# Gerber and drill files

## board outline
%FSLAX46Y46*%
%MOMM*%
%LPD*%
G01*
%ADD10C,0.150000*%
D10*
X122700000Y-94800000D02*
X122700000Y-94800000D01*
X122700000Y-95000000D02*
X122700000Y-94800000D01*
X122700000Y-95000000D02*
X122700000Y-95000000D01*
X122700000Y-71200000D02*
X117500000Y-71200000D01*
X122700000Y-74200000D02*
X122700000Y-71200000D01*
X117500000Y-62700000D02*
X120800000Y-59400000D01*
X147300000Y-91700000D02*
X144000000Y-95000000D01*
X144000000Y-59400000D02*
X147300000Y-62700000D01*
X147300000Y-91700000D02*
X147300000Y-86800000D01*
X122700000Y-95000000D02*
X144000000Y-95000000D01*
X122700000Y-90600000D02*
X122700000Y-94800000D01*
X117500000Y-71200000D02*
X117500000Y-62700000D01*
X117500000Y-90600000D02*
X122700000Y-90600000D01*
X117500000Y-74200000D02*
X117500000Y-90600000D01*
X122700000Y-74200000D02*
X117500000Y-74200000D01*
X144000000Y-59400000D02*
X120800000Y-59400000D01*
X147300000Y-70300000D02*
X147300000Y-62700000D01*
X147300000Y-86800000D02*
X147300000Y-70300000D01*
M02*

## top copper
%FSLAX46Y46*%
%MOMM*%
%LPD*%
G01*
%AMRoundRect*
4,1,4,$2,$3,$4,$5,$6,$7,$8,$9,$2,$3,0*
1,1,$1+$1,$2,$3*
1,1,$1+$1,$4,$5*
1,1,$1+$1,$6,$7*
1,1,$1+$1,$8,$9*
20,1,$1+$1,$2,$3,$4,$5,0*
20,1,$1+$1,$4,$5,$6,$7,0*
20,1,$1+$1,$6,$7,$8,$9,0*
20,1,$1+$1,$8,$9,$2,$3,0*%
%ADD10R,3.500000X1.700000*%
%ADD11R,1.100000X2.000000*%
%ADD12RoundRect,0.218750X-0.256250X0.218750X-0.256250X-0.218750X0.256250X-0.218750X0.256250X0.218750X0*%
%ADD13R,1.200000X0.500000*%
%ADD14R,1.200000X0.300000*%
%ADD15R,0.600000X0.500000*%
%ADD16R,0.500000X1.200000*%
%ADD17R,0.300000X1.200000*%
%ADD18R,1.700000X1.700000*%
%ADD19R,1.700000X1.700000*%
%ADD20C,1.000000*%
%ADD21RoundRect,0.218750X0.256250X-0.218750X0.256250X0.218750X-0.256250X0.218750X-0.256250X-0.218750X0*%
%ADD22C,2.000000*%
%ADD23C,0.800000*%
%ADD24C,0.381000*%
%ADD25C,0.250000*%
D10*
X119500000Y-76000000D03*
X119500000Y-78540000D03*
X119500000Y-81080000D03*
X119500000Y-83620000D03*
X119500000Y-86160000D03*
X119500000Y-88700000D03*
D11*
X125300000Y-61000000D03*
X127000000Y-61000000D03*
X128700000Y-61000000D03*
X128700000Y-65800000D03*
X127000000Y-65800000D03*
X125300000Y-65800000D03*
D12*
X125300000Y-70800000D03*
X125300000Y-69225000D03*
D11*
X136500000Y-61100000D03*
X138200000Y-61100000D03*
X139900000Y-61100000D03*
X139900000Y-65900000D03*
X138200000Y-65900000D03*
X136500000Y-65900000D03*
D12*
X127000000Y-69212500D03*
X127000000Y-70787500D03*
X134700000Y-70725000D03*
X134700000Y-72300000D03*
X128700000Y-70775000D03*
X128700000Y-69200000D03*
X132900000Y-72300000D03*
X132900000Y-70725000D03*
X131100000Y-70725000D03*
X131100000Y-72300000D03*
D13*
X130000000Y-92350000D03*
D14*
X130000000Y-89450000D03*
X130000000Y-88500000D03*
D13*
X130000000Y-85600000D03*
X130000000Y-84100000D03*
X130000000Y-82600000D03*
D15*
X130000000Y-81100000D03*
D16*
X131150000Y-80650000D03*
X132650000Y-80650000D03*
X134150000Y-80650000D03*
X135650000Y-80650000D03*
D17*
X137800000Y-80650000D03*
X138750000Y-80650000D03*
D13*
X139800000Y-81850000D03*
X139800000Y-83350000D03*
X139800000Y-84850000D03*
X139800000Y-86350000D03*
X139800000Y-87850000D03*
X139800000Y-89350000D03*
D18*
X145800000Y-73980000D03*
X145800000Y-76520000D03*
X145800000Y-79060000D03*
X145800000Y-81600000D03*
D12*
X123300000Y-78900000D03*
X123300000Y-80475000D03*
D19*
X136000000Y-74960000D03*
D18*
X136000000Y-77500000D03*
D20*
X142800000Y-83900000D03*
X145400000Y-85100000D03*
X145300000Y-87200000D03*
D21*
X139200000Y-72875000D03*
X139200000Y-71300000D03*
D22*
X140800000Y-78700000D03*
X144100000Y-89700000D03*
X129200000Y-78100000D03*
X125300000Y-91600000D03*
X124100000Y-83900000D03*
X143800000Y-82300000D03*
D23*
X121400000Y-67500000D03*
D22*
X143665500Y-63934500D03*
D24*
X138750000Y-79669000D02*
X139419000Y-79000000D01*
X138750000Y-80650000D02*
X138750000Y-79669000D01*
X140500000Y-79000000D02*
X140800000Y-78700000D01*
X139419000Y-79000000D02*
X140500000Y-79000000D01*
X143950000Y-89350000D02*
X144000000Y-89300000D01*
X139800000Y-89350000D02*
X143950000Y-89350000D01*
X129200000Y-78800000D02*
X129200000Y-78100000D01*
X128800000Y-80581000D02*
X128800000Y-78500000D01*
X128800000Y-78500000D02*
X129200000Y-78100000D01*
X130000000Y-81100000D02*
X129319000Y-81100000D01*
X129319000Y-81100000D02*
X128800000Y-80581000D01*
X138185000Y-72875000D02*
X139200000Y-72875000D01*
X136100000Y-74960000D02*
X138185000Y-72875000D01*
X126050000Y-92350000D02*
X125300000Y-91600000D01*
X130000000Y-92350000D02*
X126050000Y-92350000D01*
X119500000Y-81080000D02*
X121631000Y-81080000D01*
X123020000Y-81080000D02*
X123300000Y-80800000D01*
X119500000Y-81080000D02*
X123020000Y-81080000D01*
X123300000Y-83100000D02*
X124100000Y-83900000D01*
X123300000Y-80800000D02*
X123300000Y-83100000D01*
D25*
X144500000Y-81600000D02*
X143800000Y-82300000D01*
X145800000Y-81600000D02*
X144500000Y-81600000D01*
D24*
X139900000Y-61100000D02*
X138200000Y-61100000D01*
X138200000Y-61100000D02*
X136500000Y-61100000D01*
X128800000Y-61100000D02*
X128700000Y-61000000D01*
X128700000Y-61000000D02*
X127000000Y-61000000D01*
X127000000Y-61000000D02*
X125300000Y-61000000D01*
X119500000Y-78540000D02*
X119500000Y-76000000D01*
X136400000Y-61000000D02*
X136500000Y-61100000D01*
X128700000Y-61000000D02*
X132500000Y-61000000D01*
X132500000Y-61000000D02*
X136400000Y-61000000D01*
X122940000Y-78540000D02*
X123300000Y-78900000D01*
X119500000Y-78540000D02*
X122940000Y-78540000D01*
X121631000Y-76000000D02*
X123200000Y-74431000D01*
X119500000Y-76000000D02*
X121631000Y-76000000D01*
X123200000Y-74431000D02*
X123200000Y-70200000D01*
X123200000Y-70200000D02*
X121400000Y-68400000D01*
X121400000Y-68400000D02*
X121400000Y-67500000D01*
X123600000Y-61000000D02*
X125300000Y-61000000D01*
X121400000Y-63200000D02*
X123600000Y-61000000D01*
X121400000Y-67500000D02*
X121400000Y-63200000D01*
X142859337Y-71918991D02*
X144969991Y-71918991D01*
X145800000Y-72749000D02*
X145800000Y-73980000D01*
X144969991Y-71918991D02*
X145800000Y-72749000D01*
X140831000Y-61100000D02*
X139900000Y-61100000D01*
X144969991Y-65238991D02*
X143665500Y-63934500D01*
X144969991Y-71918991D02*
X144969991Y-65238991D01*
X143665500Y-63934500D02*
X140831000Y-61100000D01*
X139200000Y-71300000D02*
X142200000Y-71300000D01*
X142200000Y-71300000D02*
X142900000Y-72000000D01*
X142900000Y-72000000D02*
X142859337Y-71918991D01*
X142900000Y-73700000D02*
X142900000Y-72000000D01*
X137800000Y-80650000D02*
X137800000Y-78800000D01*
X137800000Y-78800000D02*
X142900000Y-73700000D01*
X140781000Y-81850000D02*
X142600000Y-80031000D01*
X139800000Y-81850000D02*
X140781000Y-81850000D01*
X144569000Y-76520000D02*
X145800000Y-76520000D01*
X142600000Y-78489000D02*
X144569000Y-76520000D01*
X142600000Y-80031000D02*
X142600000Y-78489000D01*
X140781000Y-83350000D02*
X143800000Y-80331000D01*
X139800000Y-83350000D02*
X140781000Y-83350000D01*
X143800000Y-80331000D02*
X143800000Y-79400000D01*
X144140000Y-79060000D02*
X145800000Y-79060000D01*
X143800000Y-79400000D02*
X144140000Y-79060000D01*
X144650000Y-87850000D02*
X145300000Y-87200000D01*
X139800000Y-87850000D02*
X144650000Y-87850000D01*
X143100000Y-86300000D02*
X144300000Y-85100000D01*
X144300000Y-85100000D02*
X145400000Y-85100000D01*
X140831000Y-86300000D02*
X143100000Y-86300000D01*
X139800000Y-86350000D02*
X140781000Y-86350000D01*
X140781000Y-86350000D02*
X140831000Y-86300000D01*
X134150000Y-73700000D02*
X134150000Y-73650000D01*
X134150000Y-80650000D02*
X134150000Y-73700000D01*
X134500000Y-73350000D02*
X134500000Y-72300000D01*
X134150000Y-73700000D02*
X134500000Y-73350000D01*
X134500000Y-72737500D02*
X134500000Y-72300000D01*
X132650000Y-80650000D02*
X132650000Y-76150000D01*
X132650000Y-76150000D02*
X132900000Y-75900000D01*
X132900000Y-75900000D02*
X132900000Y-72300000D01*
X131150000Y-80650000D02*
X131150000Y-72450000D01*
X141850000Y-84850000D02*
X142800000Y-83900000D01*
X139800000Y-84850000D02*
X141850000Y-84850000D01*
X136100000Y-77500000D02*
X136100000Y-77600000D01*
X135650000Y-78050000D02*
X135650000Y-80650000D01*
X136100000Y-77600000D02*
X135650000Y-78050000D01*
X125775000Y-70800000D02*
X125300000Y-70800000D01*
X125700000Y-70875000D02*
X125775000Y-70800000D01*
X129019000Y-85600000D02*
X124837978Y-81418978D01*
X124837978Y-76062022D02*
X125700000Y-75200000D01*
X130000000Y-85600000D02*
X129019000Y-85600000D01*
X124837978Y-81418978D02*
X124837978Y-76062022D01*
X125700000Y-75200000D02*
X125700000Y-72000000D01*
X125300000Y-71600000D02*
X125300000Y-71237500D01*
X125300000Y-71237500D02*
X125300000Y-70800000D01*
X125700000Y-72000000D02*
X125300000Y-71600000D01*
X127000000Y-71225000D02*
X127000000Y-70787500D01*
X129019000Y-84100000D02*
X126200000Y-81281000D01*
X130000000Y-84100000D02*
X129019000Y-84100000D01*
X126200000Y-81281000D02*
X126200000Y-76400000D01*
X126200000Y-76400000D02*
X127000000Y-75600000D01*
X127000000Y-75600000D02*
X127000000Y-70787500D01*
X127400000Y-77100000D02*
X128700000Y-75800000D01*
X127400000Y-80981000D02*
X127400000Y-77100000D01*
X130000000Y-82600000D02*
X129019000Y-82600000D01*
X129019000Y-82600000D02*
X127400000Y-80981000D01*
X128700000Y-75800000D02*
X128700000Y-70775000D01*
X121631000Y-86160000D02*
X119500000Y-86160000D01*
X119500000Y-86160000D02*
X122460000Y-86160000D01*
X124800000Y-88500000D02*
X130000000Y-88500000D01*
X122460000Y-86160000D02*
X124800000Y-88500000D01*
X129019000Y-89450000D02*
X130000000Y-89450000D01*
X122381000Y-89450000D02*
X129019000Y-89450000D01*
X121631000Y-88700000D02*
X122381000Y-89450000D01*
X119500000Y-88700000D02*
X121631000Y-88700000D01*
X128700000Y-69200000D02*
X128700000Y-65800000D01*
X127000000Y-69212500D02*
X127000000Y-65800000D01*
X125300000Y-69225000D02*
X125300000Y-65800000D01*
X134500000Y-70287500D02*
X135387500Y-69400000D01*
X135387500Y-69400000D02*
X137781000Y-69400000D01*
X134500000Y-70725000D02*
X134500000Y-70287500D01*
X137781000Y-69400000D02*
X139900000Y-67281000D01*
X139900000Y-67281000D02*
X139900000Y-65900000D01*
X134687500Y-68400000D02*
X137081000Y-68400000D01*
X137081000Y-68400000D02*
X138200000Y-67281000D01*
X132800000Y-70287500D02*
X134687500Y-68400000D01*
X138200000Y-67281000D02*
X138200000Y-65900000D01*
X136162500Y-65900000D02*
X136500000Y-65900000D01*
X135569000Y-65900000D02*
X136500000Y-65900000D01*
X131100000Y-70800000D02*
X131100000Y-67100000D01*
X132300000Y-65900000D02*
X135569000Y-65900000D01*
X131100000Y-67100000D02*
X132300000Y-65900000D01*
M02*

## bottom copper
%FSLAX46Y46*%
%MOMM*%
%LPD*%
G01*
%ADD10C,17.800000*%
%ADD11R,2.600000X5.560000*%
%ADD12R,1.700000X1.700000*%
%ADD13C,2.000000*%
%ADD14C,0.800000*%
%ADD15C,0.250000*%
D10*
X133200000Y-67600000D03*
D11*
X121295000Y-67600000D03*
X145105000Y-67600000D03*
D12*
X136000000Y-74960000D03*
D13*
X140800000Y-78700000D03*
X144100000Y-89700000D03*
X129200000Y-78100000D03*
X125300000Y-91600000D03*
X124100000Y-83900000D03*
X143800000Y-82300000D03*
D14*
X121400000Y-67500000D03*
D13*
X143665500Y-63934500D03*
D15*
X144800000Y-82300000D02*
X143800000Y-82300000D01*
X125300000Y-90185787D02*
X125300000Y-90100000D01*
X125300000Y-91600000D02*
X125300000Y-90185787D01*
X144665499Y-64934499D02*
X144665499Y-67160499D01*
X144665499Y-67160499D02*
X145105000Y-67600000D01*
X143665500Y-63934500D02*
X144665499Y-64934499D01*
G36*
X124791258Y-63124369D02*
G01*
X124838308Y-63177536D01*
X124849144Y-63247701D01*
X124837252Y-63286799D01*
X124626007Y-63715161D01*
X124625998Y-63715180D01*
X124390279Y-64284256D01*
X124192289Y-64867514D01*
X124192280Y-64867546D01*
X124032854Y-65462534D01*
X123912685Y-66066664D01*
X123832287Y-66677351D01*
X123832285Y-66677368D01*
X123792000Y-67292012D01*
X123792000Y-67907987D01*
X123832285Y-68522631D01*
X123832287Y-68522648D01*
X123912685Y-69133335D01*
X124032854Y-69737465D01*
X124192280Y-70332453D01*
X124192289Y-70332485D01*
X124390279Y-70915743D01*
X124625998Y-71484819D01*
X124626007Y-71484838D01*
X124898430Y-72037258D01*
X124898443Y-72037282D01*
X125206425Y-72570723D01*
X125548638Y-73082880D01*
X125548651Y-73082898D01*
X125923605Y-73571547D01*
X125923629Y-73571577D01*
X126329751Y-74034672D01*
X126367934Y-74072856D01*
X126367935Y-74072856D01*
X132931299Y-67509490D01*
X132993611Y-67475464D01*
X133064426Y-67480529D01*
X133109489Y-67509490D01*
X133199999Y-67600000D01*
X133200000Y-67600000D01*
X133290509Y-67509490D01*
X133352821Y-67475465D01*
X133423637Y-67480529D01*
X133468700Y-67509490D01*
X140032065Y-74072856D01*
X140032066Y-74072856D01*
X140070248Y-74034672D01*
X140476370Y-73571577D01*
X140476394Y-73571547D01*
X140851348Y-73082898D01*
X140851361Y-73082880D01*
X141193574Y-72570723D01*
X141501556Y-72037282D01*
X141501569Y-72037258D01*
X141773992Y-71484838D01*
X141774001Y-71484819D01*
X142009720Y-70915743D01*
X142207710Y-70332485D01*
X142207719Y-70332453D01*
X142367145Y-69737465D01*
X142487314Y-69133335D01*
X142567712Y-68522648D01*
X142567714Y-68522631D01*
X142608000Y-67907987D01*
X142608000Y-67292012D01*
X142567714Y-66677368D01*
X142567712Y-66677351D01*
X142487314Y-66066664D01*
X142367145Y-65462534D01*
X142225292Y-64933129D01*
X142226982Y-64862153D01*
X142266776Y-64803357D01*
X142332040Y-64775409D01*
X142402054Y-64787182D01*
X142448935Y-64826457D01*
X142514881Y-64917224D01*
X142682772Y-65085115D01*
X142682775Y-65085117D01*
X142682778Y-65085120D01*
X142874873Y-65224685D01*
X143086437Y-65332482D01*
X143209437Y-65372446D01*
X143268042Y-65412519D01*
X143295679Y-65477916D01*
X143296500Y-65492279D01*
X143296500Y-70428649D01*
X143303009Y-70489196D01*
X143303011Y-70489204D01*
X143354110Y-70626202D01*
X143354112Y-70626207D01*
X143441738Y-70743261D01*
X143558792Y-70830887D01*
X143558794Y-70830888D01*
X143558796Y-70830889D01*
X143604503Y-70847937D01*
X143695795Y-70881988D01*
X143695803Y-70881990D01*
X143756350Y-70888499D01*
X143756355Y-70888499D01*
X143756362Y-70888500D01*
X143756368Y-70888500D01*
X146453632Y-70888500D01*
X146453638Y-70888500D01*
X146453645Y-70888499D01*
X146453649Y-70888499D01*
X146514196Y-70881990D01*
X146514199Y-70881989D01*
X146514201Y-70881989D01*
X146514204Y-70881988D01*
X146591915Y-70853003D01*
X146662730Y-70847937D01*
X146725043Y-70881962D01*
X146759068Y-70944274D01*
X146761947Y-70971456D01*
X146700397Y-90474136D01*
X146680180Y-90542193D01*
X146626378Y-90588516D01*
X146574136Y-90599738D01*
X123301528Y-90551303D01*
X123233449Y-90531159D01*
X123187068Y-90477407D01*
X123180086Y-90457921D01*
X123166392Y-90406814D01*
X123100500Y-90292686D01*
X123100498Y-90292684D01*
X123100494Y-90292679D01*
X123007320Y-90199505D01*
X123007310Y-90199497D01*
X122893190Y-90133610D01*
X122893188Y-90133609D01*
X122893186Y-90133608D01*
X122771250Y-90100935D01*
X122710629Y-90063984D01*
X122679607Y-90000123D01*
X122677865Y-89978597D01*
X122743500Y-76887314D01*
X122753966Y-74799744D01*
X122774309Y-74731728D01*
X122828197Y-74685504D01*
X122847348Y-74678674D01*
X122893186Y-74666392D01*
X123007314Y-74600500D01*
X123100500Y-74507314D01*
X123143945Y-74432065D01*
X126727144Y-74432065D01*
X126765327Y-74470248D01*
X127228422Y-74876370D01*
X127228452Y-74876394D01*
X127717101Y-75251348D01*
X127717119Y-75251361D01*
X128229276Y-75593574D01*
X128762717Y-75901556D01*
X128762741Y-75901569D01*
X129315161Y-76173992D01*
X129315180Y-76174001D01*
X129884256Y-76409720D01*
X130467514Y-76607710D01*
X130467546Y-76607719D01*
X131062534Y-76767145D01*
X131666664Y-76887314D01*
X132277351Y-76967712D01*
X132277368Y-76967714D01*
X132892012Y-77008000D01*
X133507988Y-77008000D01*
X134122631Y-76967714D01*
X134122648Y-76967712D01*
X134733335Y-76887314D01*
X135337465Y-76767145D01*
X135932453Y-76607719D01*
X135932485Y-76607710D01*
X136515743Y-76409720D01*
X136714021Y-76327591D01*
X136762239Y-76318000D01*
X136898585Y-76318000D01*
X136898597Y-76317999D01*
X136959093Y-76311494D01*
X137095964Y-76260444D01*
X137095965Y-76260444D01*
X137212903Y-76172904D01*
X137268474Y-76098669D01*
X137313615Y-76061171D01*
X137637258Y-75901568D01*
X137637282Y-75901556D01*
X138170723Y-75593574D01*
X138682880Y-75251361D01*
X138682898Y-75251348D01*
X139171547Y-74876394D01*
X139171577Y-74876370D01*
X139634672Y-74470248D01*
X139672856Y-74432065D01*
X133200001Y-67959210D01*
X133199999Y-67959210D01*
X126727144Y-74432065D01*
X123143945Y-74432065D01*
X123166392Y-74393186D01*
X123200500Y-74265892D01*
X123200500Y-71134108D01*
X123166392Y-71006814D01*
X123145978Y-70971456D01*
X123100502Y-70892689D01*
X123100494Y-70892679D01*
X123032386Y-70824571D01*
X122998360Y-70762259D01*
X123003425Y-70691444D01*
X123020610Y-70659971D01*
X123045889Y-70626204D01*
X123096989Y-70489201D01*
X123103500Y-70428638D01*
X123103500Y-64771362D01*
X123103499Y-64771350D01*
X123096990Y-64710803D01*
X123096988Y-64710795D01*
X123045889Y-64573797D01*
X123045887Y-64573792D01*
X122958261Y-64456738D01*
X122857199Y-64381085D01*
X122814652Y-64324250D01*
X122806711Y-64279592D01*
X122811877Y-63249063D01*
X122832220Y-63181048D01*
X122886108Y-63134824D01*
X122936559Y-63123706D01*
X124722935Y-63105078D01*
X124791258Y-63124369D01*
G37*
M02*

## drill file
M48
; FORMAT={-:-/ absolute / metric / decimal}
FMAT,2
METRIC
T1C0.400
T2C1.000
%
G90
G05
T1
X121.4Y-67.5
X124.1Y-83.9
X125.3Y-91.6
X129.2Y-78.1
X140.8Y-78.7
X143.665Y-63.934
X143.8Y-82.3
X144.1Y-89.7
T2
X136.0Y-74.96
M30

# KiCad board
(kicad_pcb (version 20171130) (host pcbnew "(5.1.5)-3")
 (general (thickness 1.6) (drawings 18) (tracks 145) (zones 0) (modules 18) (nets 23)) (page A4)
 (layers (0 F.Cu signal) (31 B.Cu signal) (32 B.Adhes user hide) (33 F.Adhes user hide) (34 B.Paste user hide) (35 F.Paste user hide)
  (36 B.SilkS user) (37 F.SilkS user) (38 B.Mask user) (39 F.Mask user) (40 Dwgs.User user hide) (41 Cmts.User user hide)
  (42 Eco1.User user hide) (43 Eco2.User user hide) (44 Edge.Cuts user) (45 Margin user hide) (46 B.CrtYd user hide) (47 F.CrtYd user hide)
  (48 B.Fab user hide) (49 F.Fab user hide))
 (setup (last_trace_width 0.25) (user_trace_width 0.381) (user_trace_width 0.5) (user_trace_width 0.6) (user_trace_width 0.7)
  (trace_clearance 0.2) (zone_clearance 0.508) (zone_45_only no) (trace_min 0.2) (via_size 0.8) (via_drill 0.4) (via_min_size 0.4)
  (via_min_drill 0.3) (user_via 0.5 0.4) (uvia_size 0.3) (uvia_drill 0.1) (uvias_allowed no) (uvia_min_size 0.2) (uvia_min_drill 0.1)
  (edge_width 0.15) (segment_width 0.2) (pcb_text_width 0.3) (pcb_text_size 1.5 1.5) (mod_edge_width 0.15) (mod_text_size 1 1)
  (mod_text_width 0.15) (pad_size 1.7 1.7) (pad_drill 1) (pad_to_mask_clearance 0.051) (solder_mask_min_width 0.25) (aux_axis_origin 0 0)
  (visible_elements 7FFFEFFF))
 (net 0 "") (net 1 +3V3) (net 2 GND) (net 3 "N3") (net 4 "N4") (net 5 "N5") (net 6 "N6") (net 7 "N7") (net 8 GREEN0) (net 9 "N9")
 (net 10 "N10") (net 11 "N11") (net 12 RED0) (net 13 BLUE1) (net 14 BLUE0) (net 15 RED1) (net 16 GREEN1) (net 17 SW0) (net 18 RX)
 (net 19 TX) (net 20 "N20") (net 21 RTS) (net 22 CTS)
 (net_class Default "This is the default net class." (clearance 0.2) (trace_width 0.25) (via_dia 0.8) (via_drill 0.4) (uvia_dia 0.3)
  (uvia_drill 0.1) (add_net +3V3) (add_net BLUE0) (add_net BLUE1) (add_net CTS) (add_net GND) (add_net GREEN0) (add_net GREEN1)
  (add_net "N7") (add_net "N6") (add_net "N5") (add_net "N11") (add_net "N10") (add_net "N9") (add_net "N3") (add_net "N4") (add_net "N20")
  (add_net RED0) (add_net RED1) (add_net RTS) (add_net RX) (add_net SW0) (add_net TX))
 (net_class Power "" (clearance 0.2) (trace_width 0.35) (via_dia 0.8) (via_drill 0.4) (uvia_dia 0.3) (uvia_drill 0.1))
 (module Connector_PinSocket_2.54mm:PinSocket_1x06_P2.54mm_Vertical (layer F.Cu) (at 119.5 76)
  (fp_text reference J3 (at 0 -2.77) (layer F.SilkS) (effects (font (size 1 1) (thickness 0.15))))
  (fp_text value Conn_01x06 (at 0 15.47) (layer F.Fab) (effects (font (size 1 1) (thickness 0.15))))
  (pad 1 smd rect (at 0 0) (size 3.5 1.7) (layers F.Cu F.Paste F.Mask) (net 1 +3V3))
  (pad 2 smd rect (at 0 2.54) (size 3.5 1.7) (layers F.Cu F.Paste F.Mask) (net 1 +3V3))
  (pad 3 smd rect (at 0 5.08) (size 3.5 1.7) (layers F.Cu F.Paste F.Mask) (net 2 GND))
  (pad 4 smd rect (at 0 7.62) (size 3.5 1.7) (layers F.Cu F.Paste F.Mask))
  (pad 5 smd rect (at 0 10.16) (size 3.5 1.7) (layers F.Cu F.Paste F.Mask) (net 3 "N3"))
  (pad 6 smd rect (at 0 12.7) (size 3.5 1.7) (layers F.Cu F.Paste F.Mask) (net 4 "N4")))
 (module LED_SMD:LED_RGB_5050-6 (layer F.Cu) (at 127 63.4 90)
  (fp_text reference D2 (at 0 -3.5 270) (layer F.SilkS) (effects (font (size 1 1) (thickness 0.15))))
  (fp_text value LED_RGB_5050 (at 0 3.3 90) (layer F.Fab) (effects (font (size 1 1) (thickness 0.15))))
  (pad 6 smd rect (at 2.4 -1.7 180) (size 1.1 2) (layers F.Cu F.Paste F.Mask) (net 1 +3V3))
  (pad 5 smd rect (at 2.4 0 180) (size 1.1 2) (layers F.Cu F.Paste F.Mask) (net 1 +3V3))
  (pad 4 smd rect (at 2.4 1.7 180) (size 1.1 2) (layers F.Cu F.Paste F.Mask) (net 1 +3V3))
  (pad 3 smd rect (at -2.4 1.7 180) (size 1.1 2) (layers F.Cu F.Paste F.Mask) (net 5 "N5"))
  (pad 2 smd rect (at -2.4 0 180) (size 1.1 2) (layers F.Cu F.Paste F.Mask) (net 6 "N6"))
  (pad 1 smd rect (at -2.4 -1.7 180) (size 1.1 2) (layers F.Cu F.Paste F.Mask) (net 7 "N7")))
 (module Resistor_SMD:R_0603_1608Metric (layer F.Cu) (at 125.3 70.0125 270)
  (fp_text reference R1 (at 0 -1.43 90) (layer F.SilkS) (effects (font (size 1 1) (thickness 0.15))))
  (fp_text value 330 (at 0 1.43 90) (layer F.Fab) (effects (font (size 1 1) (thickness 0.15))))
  (pad 2 smd roundrect (at 0.7875 0 270) (size 0.875 0.95) (layers F.Cu F.Paste F.Mask) (roundrect_rratio 0.25) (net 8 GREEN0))
  (pad 1 smd roundrect (at -0.7875 0 270) (size 0.875 0.95) (layers F.Cu F.Paste F.Mask) (roundrect_rratio 0.25) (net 7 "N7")))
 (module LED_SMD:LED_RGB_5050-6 (layer F.Cu) (at 138.2 63.5 90)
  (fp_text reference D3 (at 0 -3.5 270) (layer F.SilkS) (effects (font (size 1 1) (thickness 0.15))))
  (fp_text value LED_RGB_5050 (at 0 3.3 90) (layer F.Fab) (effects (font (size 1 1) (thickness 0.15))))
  (pad 6 smd rect (at 2.4 -1.7 180) (size 1.1 2) (layers F.Cu F.Paste F.Mask) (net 1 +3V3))
  (pad 5 smd rect (at 2.4 0 180) (size 1.1 2) (layers F.Cu F.Paste F.Mask) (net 1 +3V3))
  (pad 4 smd rect (at 2.4 1.7 180) (size 1.1 2) (layers F.Cu F.Paste F.Mask) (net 1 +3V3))
  (pad 3 smd rect (at -2.4 1.7 180) (size 1.1 2) (layers F.Cu F.Paste F.Mask) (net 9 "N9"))
  (pad 2 smd rect (at -2.4 0 180) (size 1.1 2) (layers F.Cu F.Paste F.Mask) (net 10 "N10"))
  (pad 1 smd rect (at -2.4 -1.7 180) (size 1.1 2) (layers F.Cu F.Paste F.Mask) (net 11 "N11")))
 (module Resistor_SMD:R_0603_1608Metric (layer F.Cu) (at 127 70 270)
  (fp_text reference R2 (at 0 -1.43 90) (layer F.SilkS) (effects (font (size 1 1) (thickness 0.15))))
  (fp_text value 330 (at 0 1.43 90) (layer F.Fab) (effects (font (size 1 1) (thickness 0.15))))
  (pad 1 smd roundrect (at -0.7875 0 270) (size 0.875 0.95) (layers F.Cu F.Paste F.Mask) (roundrect_rratio 0.25) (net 6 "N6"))
  (pad 2 smd roundrect (at 0.7875 0 270) (size 0.875 0.95) (layers F.Cu F.Paste F.Mask) (roundrect_rratio 0.25) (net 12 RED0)))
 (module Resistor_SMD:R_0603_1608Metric (layer F.Cu) (at 134.7 71.5125 270)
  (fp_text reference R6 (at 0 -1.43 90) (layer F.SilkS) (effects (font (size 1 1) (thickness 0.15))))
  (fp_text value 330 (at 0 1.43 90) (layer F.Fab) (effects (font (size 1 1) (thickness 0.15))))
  (pad 1 smd roundrect (at -0.7875 0 270) (size 0.875 0.95) (layers F.Cu F.Paste F.Mask) (roundrect_rratio 0.25) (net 9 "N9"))
  (pad 2 smd roundrect (at 0.7875 0 270) (size 0.875 0.95) (layers F.Cu F.Paste F.Mask) (roundrect_rratio 0.25) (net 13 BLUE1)))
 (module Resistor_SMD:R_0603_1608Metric (layer F.Cu) (at 128.7 69.9875 270)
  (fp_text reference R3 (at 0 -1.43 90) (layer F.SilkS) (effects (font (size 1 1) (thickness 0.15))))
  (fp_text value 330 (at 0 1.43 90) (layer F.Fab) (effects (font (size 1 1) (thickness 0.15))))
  (pad 2 smd roundrect (at 0.7875 0 270) (size 0.875 0.95) (layers F.Cu F.Paste F.Mask) (roundrect_rratio 0.25) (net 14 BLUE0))
  (pad 1 smd roundrect (at -0.7875 0 270) (size 0.875 0.95) (layers F.Cu F.Paste F.Mask) (roundrect_rratio 0.25) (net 5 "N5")))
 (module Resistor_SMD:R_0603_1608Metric (layer F.Cu) (at 132.9 71.5125 270)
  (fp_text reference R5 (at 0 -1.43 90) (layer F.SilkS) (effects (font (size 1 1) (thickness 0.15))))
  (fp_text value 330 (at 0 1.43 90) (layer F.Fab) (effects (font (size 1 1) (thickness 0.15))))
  (pad 2 smd roundrect (at 0.7875 0 270) (size 0.875 0.95) (layers F.Cu F.Paste F.Mask) (roundrect_rratio 0.25) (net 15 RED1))
  (pad 1 smd roundrect (at -0.7875 0 270) (size 0.875 0.95) (layers F.Cu F.Paste F.Mask) (roundrect_rratio 0.25) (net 10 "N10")))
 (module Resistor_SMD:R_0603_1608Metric (layer F.Cu) (at 131.1 71.5125 270)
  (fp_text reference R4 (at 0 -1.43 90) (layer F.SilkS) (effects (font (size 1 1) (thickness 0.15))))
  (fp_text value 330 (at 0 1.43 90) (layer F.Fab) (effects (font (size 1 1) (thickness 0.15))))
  (pad 1 smd roundrect (at -0.7875 0 270) (size 0.875 0.95) (layers F.Cu F.Paste F.Mask) (roundrect_rratio 0.25) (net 11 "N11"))
  (pad 2 smd roundrect (at 0.7875 0 270) (size 0.875 0.95) (layers F.Cu F.Paste F.Mask) (roundrect_rratio 0.25) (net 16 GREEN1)))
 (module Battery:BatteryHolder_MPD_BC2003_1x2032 (layer B.Cu) (at 133.2 67.6 180)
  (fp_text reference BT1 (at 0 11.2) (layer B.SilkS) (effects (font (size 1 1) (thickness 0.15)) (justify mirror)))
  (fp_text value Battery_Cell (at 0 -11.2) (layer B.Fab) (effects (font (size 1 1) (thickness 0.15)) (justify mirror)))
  (pad 2 smd circle (at 0 0 180) (size 17.8 17.8) (layers B.Cu B.Mask) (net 2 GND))
  (pad 1 smd rect (at 11.905 0 180) (size 2.6 5.56) (layers B.Cu B.Paste B.Mask) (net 1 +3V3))
  (pad 1 smd rect (at -11.905 0 180) (size 2.6 5.56) (layers B.Cu B.Paste B.Mask) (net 1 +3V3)))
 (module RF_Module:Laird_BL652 (layer F.Cu) (at 134.9 86.5 90)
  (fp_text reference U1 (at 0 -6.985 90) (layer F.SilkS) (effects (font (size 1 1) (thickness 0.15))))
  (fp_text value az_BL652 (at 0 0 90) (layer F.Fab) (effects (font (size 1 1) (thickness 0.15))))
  (pad 1 smd rect (at -5.85 -4.9 180) (size 1.2 0.5) (layers F.Cu F.Paste F.Mask) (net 2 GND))
  (pad 5 smd rect (at -2.95 -4.9 180) (size 1.2 0.3) (layers F.Cu F.Paste F.Mask) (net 4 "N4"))
  (pad 6 smd rect (at -2 -4.9 180) (size 1.2 0.3) (layers F.Cu F.Paste F.Mask) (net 3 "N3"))
  (pad 10 smd rect (at 0.9 -4.9 180) (size 1.2 0.5) (layers F.Cu F.Paste F.Mask) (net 8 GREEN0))
  (pad 12 smd rect (at 2.4 -4.9 180) (size 1.2 0.5) (layers F.Cu F.Paste F.Mask) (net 12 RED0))
  (pad 14 smd rect (at 3.9 -4.9 180) (size 1.2 0.5) (layers F.Cu F.Paste F.Mask) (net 14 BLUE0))
  (pad 16 smd rect (at 5.4 -4.9 180) (size 0.6 0.5) (layers F.Cu F.Paste F.Mask) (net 2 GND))
  (pad 17 smd rect (at 5.85 -3.75 90) (size 1.2 0.5) (layers F.Cu F.Paste F.Mask) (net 16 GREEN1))
  (pad 19 smd rect (at 5.85 -2.25 90) (size 1.2 0.5) (layers F.Cu F.Paste F.Mask) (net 15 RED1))
  (pad 21 smd rect (at 5.85 -0.75 90) (size 1.2 0.5) (layers F.Cu F.Paste F.Mask) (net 13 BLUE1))
  (pad 23 smd rect (at 5.85 0.75 90) (size 1.2 0.5) (layers F.Cu F.Paste F.Mask) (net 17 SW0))
  (pad 26 smd rect (at 5.85 2.9 90) (size 1.2 0.3) (layers F.Cu F.Paste F.Mask) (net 1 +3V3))
  (pad 27 smd rect (at 5.85 3.85 90) (size 1.2 0.3) (layers F.Cu F.Paste F.Mask) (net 2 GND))
  (pad 29 smd rect (at 4.65 4.9 180) (size 1.2 0.5) (layers F.Cu F.Paste F.Mask) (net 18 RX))
  (pad 31 smd rect (at 3.15 4.9 180) (size 1.2 0.5) (layers F.Cu F.Paste F.Mask) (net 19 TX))
  (pad 33 smd rect (at 1.65 4.9 180) (size 1.2 0.5) (layers F.Cu F.Paste F.Mask) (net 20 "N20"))
  (pad 35 smd rect (at 0.15 4.9 180) (size 1.2 0.5) (layers F.Cu F.Paste F.Mask) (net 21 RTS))
  (pad 37 smd rect (at -1.35 4.9 180) (size 1.2 0.5) (layers F.Cu F.Paste F.Mask) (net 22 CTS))
  (pad 39 smd rect (at -2.85 4.9 180) (size 1.2 0.5) (layers F.Cu F.Paste F.Mask) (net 2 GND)))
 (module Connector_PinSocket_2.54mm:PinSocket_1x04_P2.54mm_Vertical (layer F.Cu) (at 145.8 73.98)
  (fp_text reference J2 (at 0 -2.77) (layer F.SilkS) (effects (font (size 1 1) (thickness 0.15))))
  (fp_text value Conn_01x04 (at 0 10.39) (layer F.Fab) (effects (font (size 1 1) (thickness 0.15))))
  (pad 1 smd rect (at 0 0) (size 1.7 1.7) (layers F.Cu F.Paste F.Mask) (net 1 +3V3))
  (pad 2 smd rect (at 0 2.54) (size 1.7 1.7) (layers F.Cu F.Paste F.Mask) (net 18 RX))
  (pad 3 smd rect (at 0 5.08) (size 1.7 1.7) (layers F.Cu F.Paste F.Mask) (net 19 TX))
  (pad 4 smd rect (at 0 7.62) (size 1.7 1.7) (layers F.Cu F.Paste F.Mask) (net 2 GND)))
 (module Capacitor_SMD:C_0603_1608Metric (layer F.Cu) (at 123.3 79.6875 270)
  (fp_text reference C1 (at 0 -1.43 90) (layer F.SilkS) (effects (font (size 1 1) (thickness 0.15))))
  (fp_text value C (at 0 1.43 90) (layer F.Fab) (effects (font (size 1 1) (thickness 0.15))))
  (pad 1 smd roundrect (at -0.7875 0 270) (size 0.875 0.95) (layers F.Cu F.Paste F.Mask) (roundrect_rratio 0.25) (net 1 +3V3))
  (pad 2 smd roundrect (at 0.7875 0 270) (size 0.875 0.95) (layers F.Cu F.Paste F.Mask) (roundrect_rratio 0.25) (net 2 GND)))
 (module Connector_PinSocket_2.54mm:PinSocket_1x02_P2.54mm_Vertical (layer F.Cu) (at 136 77.5 180)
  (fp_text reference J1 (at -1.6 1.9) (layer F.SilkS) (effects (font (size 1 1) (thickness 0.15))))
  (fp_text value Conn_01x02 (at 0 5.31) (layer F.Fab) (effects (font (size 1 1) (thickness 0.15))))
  (pad 2 thru_hole rect (at 0 2.54 180) (size 1.7 1.7) (drill 1) (layers *.Cu *.Mask) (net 2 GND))
  (pad 1 smd rect (at 0 0 180) (size 1.7 1.7) (layers F.Cu F.Paste F.Mask) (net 17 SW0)))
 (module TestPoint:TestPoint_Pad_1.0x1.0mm (layer F.Cu) (at 142.8 83.9)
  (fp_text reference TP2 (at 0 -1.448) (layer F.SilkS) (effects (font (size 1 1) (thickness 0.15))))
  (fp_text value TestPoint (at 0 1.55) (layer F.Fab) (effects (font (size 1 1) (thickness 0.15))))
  (pad 1 smd circle (at 0 0) (size 1 1) (layers F.Cu F.Mask) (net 20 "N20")))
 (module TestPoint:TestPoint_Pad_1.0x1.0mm (layer F.Cu) (at 145.4 85.1)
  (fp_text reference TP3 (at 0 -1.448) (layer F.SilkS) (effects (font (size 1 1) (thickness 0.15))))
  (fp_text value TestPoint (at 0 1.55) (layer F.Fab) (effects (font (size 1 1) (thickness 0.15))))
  (pad 1 smd circle (at 0 0) (size 1 1) (layers F.Cu F.Mask) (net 21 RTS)))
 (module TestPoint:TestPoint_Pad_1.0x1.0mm (layer F.Cu) (at 145.3 87.2)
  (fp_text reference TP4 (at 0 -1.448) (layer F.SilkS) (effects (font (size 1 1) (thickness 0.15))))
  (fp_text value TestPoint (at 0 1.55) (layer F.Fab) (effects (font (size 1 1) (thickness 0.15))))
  (pad 1 smd circle (at 0 0) (size 1 1) (layers F.Cu F.Mask) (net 22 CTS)))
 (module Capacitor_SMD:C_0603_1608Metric (layer F.Cu) (at 139.2 72.0875 90)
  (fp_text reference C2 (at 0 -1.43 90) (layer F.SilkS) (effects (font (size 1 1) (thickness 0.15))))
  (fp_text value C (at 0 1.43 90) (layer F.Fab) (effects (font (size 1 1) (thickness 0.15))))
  (pad 1 smd roundrect (at -0.7875 0 90) (size 0.875 0.95) (layers F.Cu F.Paste F.Mask) (roundrect_rratio 0.25) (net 2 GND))
  (pad 2 smd roundrect (at 0.7875 0 90) (size 0.875 0.95) (layers F.Cu F.Paste F.Mask) (roundrect_rratio 0.25) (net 1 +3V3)))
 (gr_line (start 122.7 94.8) (end 122.7 94.8) (layer Edge.Cuts) (width 0.15))
 (gr_line (start 122.7 95) (end 122.7 94.8) (layer Edge.Cuts) (width 0.15))
 (gr_line (start 122.7 95) (end 122.7 95) (layer Edge.Cuts) (width 0.15))
 (gr_line (start 122.7 71.2) (end 117.5 71.2) (layer Edge.Cuts) (width 0.15))
 (gr_line (start 122.7 74.2) (end 122.7 71.2) (layer Edge.Cuts) (width 0.15))
 (gr_line (start 117.5 62.7) (end 120.8 59.4) (layer Edge.Cuts) (width 0.15))
 (gr_line (start 147.3 91.7) (end 144 95) (layer Edge.Cuts) (width 0.15))
 (gr_line (start 144 59.4) (end 147.3 62.7) (layer Edge.Cuts) (width 0.15))
 (gr_line (start 147.3 91.7) (end 147.3 86.8) (layer Edge.Cuts) (width 0.15))
 (gr_line (start 122.7 95) (end 144 95) (layer Edge.Cuts) (width 0.15))
 (gr_line (start 122.7 90.6) (end 122.7 94.8) (layer Edge.Cuts) (width 0.15))
 (gr_line (start 117.5 71.2) (end 117.5 62.7) (layer Edge.Cuts) (width 0.15))
 (gr_line (start 117.5 90.6) (end 122.7 90.6) (layer Edge.Cuts) (width 0.15))
 (gr_line (start 117.5 74.2) (end 117.5 90.6) (layer Edge.Cuts) (width 0.15))
 (gr_line (start 122.7 74.2) (end 117.5 74.2) (layer Edge.Cuts) (width 0.15))
 (gr_line (start 144 59.4) (end 120.8 59.4) (layer Edge.Cuts) (width 0.15))
 (gr_line (start 147.3 70.3) (end 147.3 62.7) (layer Edge.Cuts) (width 0.15))
 (gr_line (start 147.3 86.8) (end 147.3 70.3) (layer Edge.Cuts) (width 0.15))
 (via (at 140.8 78.7) (size 2) (drill 0.4) (layers F.Cu B.Cu) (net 2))
 (segment (start 138.75 79.669) (end 139.419 79) (width 0.381) (layer F.Cu) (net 2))
 (segment (start 138.75 80.65) (end 138.75 79.669) (width 0.381) (layer F.Cu) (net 2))
 (segment (start 140.5 79) (end 140.8 78.7) (width 0.381) (layer F.Cu) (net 2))
 (segment (start 139.419 79) (end 140.5 79) (width 0.381) (layer F.Cu) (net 2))
 (via (at 144.1 89.7) (size 2) (drill 0.4) (layers F.Cu B.Cu) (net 2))
 (segment (start 143.95 89.35) (end 144 89.3) (width 0.381) (layer F.Cu) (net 2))
 (segment (start 139.8 89.35) (end 143.95 89.35) (width 0.381) (layer F.Cu) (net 2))
 (segment (start 129.2 78.8) (end 129.2 78.1) (width 0.381) (layer F.Cu) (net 2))
 (via (at 129.2 78.1) (size 2) (drill 0.4) (layers F.Cu B.Cu) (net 2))
 (segment (start 128.8 80.581) (end 128.8 78.5) (width 0.381) (layer F.Cu) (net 2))
 (segment (start 128.8 78.5) (end 129.2 78.1) (width 0.381) (layer F.Cu) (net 2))
 (segment (start 130 81.1) (end 129.319 81.1) (width 0.381) (layer F.Cu) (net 2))
 (segment (start 129.319 81.1) (end 128.8 80.581) (width 0.381) (layer F.Cu) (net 2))
 (segment (start 138.185 72.875) (end 139.2 72.875) (width 0.381) (layer F.Cu) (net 2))
 (segment (start 136.1 74.96) (end 138.185 72.875) (width 0.381) (layer F.Cu) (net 2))
 (segment (start 126.05 92.35) (end 125.3 91.6) (width 0.381) (layer F.Cu) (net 2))
 (via (at 125.3 91.6) (size 2) (drill 0.4) (layers F.Cu B.Cu) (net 2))
 (segment (start 130 92.35) (end 126.05 92.35) (width 0.381) (layer F.Cu) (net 2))
 (segment (start 119.5 81.08) (end 121.631 81.08) (width 0.381) (layer F.Cu) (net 2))
 (via (at 124.1 83.9) (size 2) (drill 0.4) (layers F.Cu B.Cu) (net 2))
 (segment (start 123.02 81.08) (end 123.3 80.8) (width 0.381) (layer F.Cu) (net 2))
 (segment (start 119.5 81.08) (end 123.02 81.08) (width 0.381) (layer F.Cu) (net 2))
 (segment (start 123.3 83.1) (end 124.1 83.9) (width 0.381) (layer F.Cu) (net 2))
 (segment (start 123.3 80.8) (end 123.3 83.1) (width 0.381) (layer F.Cu) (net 2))
 (via (at 143.8 82.3) (size 2) (drill 0.4) (layers F.Cu B.Cu) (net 2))
 (segment (start 144.8 82.3) (end 143.8 82.3) (width 0.25) (layer B.Cu) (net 2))
 (segment (start 144.5 81.6) (end 143.8 82.3) (width 0.25) (layer F.Cu) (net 2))
 (segment (start 145.8 81.6) (end 144.5 81.6) (width 0.25) (layer F.Cu) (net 2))
 (segment (start 125.3 90.185787) (end 125.3 90.1) (width 0.25) (layer B.Cu) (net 2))
 (segment (start 125.3 91.6) (end 125.3 90.185787) (width 0.25) (layer B.Cu) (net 2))
 (segment (start 139.9 61.1) (end 138.2 61.1) (width 0.381) (layer F.Cu) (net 1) (status 30))
 (segment (start 138.2 61.1) (end 136.5 61.1) (width 0.381) (layer F.Cu) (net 1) (status 30))
 (segment (start 128.8 61.1) (end 128.7 61) (width 0.381) (layer F.Cu) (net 1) (status 30))
 (segment (start 128.7 61) (end 127 61) (width 0.381) (layer F.Cu) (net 1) (status 30))
 (segment (start 127 61) (end 125.3 61) (width 0.381) (layer F.Cu) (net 1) (status 30))
 (segment (start 119.5 78.54) (end 119.5 76) (width 0.381) (layer F.Cu) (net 1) (status 30))
 (segment (start 136.4 61) (end 136.5 61.1) (width 0.381) (layer F.Cu) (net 1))
 (segment (start 128.7 61) (end 132.5 61) (width 0.381) (layer F.Cu) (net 1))
 (segment (start 132.5 61) (end 136.4 61) (width 0.381) (layer F.Cu) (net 1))
 (segment (start 122.94 78.54) (end 123.3 78.9) (width 0.381) (layer F.Cu) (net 1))
 (segment (start 119.5 78.54) (end 122.94 78.54) (width 0.381) (layer F.Cu) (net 1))
 (segment (start 121.631 76) (end 123.2 74.431) (width 0.381) (layer F.Cu) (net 1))
 (segment (start 119.5 76) (end 121.631 76) (width 0.381) (layer F.Cu) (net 1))
 (segment (start 123.2 74.431) (end 123.2 70.2) (width 0.381) (layer F.Cu) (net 1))
 (segment (start 123.2 70.2) (end 121.4 68.4) (width 0.381) (layer F.Cu) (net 1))
 (segment (start 121.4 68.4) (end 121.4 67.5) (width 0.381) (layer F.Cu) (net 1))
 (segment (start 123.6 61) (end 125.3 61) (width 0.381) (layer F.Cu) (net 1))
 (segment (start 121.4 63.2) (end 123.6 61) (width 0.381) (layer F.Cu) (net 1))
 (segment (start 121.4 67.5) (end 121.4 63.2) (width 0.381) (layer F.Cu) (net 1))
 (via (at 121.4 67.5) (size 0.8) (drill 0.4) (layers F.Cu B.Cu) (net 1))
 (segment (start 142.859337 71.918991) (end 144.969991 71.918991) (width 0.381) (layer F.Cu) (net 1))
 (segment (start 145.8 72.749) (end 145.8 73.98) (width 0.381) (layer F.Cu) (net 1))
 (segment (start 144.969991 71.918991) (end 145.8 72.749) (width 0.381) (layer F.Cu) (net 1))
 (segment (start 140.831 61.1) (end 139.9 61.1) (width 0.381) (layer F.Cu) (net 1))
 (segment (start 144.969991 65.238991) (end 143.6655 63.9345) (width 0.381) (layer F.Cu) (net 1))
 (segment (start 144.969991 71.918991) (end 144.969991 65.238991) (width 0.381) (layer F.Cu) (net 1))
 (segment (start 143.6655 63.9345) (end 140.831 61.1) (width 0.381) (layer F.Cu) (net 1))
 (via (at 143.6655 63.9345) (size 2) (drill 0.4) (layers F.Cu B.Cu) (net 1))
 (segment (start 139.2 71.3) (end 142.2 71.3) (width 0.381) (layer F.Cu) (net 1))
 (segment (start 142.2 71.3) (end 142.9 72) (width 0.381) (layer F.Cu) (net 1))
 (segment (start 142.9 72) (end 142.859337 71.918991) (width 0.381) (layer F.Cu) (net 1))
 (segment (start 142.9 73.7) (end 142.9 72) (width 0.381) (layer F.Cu) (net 1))
 (segment (start 137.8 80.65) (end 137.8 78.8) (width 0.381) (layer F.Cu) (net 1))
 (segment (start 137.8 78.8) (end 142.9 73.7) (width 0.381) (layer F.Cu) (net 1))
 (segment (start 144.665499 64.934499) (end 144.665499 67.160499) (width 0.25) (layer B.Cu) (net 1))
 (segment (start 144.665499 67.160499) (end 145.105 67.6) (width 0.25) (layer B.Cu) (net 1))
 (segment (start 143.6655 63.9345) (end 144.665499 64.934499) (width 0.25) (layer B.Cu) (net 1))
 (segment (start 140.781 81.85) (end 142.6 80.031) (width 0.381) (layer F.Cu) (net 18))
 (segment (start 139.8 81.85) (end 140.781 81.85) (width 0.381) (layer F.Cu) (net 18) (status 10))
 (segment (start 144.569 76.52) (end 145.8 76.52) (width 0.381) (layer F.Cu) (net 18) (status 20))
 (segment (start 142.6 78.489) (end 144.569 76.52) (width 0.381) (layer F.Cu) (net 18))
 (segment (start 142.6 80.031) (end 142.6 78.489) (width 0.381) (layer F.Cu) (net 18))
 (segment (start 140.781 83.35) (end 143.8 80.331) (width 0.381) (layer F.Cu) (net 19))
 (segment (start 139.8 83.35) (end 140.781 83.35) (width 0.381) (layer F.Cu) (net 19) (status 10))
 (segment (start 143.8 80.331) (end 143.8 79.4) (width 0.381) (layer F.Cu) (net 19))
 (segment (start 144.14 79.06) (end 145.8 79.06) (width 0.381) (layer F.Cu) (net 19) (status 20))
 (segment (start 143.8 79.4) (end 144.14 79.06) (width 0.381) (layer F.Cu) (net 19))
 (segment (start 144.65 87.85) (end 145.3 87.2) (width 0.381) (layer F.Cu) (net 22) (status 20))
 (segment (start 139.8 87.85) (end 144.65 87.85) (width 0.381) (layer F.Cu) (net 22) (status 10))
 (segment (start 143.1 86.3) (end 144.3 85.1) (width 0.381) (layer F.Cu) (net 21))
 (segment (start 144.3 85.1) (end 145.4 85.1) (width 0.381) (layer F.Cu) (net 21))
 (segment (start 140.831 86.3) (end 143.1 86.3) (width 0.381) (layer F.Cu) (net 21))
 (segment (start 139.8 86.35) (end 140.781 86.35) (width 0.381) (layer F.Cu) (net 21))
 (segment (start 140.781 86.35) (end 140.831 86.3) (width 0.381) (layer F.Cu) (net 21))
 (segment (start 134.15 73.7) (end 134.15 73.65) (width 0.381) (layer F.Cu) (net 13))
 (segment (start 134.15 80.65) (end 134.15 73.7) (width 0.381) (layer F.Cu) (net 13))
 (segment (start 134.5 73.35) (end 134.5 72.3) (width 0.381) (layer F.Cu) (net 13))
 (segment (start 134.15 73.7) (end 134.5 73.35) (width 0.381) (layer F.Cu) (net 13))
 (segment (start 134.5 72.7375) (end 134.5 72.3) (width 0.381) (layer F.Cu) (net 13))
 (segment (start 132.65 80.65) (end 132.65 76.15) (width 0.381) (layer F.Cu) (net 15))
 (segment (start 132.65 76.15) (end 132.9 75.9) (width 0.381) (layer F.Cu) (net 15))
 (segment (start 132.9 75.9) (end 132.9 72.3) (width 0.381) (layer F.Cu) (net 15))
 (segment (start 131.15 80.65) (end 131.15 72.45) (width 0.381) (layer F.Cu) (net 16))
 (segment (start 141.85 84.85) (end 142.8 83.9) (width 0.381) (layer F.Cu) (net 20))
 (segment (start 139.8 84.85) (end 141.85 84.85) (width 0.381) (layer F.Cu) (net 20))
 (segment (start 136.1 77.5) (end 136.1 77.6) (width 0.381) (layer F.Cu) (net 17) (status 30))
 (segment (start 135.65 78.05) (end 135.65 80.65) (width 0.381) (layer F.Cu) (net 17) (status 30))
 (segment (start 136.1 77.6) (end 135.65 78.05) (width 0.381) (layer F.Cu) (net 17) (status 30))
 (segment (start 125.775 70.8) (end 125.3 70.8) (width 0.381) (layer F.Cu) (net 8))
 (segment (start 125.7 70.875) (end 125.775 70.8) (width 0.381) (layer F.Cu) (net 8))
 (segment (start 129.019 85.6) (end 124.837978 81.418978) (width 0.381) (layer F.Cu) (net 8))
 (segment (start 124.837978 76.062022) (end 125.7 75.2) (width 0.381) (layer F.Cu) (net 8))
 (segment (start 130 85.6) (end 129.019 85.6) (width 0.381) (layer F.Cu) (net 8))
 (segment (start 124.837978 81.418978) (end 124.837978 76.062022) (width 0.381) (layer F.Cu) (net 8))
 (segment (start 125.7 75.2) (end 125.7 72) (width 0.381) (layer F.Cu) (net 8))
 (segment (start 125.3 71.6) (end 125.3 71.2375) (width 0.381) (layer F.Cu) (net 8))
 (segment (start 125.3 71.2375) (end 125.3 70.8) (width 0.381) (layer F.Cu) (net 8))
 (segment (start 125.7 72) (end 125.3 71.6) (width 0.381) (layer F.Cu) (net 8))
 (segment (start 127 71.225) (end 127 70.7875) (width 0.381) (layer F.Cu) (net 12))
 (segment (start 129.019 84.1) (end 126.2 81.281) (width 0.381) (layer F.Cu) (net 12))
 (segment (start 130 84.1) (end 129.019 84.1) (width 0.381) (layer F.Cu) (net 12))
 (segment (start 126.2 81.281) (end 126.2 76.4) (width 0.381) (layer F.Cu) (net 12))
 (segment (start 126.2 76.4) (end 127 75.6) (width 0.381) (layer F.Cu) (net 12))
 (segment (start 127 75.6) (end 127 70.7875) (width 0.381) (layer F.Cu) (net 12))
 (segment (start 127.4 77.1) (end 128.7 75.8) (width 0.381) (layer F.Cu) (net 14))
 (segment (start 127.4 80.981) (end 127.4 77.1) (width 0.381) (layer F.Cu) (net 14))
 (segment (start 130 82.6) (end 129.019 82.6) (width 0.381) (layer F.Cu) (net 14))
 (segment (start 129.019 82.6) (end 127.4 80.981) (width 0.381) (layer F.Cu) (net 14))
 (segment (start 128.7 75.8) (end 128.7 70.775) (width 0.381) (layer F.Cu) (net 14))
 (segment (start 121.631 86.16) (end 119.5 86.16) (width 0.381) (layer F.Cu) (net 3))
 (segment (start 119.5 86.16) (end 122.46 86.16) (width 0.381) (layer F.Cu) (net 3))
 (segment (start 124.8 88.5) (end 130 88.5) (width 0.381) (layer F.Cu) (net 3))
 (segment (start 122.46 86.16) (end 124.8 88.5) (width 0.381) (layer F.Cu) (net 3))
 (segment (start 129.019 89.45) (end 130 89.45) (width 0.381) (layer F.Cu) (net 4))
 (segment (start 122.381 89.45) (end 129.019 89.45) (width 0.381) (layer F.Cu) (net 4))
 (segment (start 121.631 88.7) (end 122.381 89.45) (width 0.381) (layer F.Cu) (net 4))
 (segment (start 119.5 88.7) (end 121.631 88.7) (width 0.381) (layer F.Cu) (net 4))
 (segment (start 128.7 69.2) (end 128.7 65.8) (width 0.381) (layer F.Cu) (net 5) (status 30))
 (segment (start 127 69.2125) (end 127 65.8) (width 0.381) (layer F.Cu) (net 6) (status 30))
 (segment (start 125.3 69.225) (end 125.3 65.8) (width 0.381) (layer F.Cu) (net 7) (status 30))
 (segment (start 134.5 70.2875) (end 135.3875 69.4) (width 0.381) (layer F.Cu) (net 9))
 (segment (start 135.3875 69.4) (end 137.781 69.4) (width 0.381) (layer F.Cu) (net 9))
 (segment (start 134.5 70.725) (end 134.5 70.2875) (width 0.381) (layer F.Cu) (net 9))
 (segment (start 137.781 69.4) (end 139.9 67.281) (width 0.381) (layer F.Cu) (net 9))
 (segment (start 139.9 67.281) (end 139.9 65.9) (width 0.381) (layer F.Cu) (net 9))
 (segment (start 134.6875 68.4) (end 137.081 68.4) (width 0.381) (layer F.Cu) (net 10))
 (segment (start 137.081 68.4) (end 138.2 67.281) (width 0.381) (layer F.Cu) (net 10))
 (segment (start 132.8 70.2875) (end 134.6875 68.4) (width 0.381) (layer F.Cu) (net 10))
 (segment (start 138.2 67.281) (end 138.2 65.9) (width 0.381) (layer F.Cu) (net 10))
 (segment (start 136.1625 65.9) (end 136.5 65.9) (width 0.381) (layer F.Cu) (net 11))
 (segment (start 135.569 65.9) (end 136.5 65.9) (width 0.381) (layer F.Cu) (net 11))
 (segment (start 131.1 70.8) (end 131.1 67.1) (width 0.381) (layer F.Cu) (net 11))
 (segment (start 132.3 65.9) (end 135.569 65.9) (width 0.381) (layer F.Cu) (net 11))
 (segment (start 131.1 67.1) (end 132.3 65.9) (width 0.381) (layer F.Cu) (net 11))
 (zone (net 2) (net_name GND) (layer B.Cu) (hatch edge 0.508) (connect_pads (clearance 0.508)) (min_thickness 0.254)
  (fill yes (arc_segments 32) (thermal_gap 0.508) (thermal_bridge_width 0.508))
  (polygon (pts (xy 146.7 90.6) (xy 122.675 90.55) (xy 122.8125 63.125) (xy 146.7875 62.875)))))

